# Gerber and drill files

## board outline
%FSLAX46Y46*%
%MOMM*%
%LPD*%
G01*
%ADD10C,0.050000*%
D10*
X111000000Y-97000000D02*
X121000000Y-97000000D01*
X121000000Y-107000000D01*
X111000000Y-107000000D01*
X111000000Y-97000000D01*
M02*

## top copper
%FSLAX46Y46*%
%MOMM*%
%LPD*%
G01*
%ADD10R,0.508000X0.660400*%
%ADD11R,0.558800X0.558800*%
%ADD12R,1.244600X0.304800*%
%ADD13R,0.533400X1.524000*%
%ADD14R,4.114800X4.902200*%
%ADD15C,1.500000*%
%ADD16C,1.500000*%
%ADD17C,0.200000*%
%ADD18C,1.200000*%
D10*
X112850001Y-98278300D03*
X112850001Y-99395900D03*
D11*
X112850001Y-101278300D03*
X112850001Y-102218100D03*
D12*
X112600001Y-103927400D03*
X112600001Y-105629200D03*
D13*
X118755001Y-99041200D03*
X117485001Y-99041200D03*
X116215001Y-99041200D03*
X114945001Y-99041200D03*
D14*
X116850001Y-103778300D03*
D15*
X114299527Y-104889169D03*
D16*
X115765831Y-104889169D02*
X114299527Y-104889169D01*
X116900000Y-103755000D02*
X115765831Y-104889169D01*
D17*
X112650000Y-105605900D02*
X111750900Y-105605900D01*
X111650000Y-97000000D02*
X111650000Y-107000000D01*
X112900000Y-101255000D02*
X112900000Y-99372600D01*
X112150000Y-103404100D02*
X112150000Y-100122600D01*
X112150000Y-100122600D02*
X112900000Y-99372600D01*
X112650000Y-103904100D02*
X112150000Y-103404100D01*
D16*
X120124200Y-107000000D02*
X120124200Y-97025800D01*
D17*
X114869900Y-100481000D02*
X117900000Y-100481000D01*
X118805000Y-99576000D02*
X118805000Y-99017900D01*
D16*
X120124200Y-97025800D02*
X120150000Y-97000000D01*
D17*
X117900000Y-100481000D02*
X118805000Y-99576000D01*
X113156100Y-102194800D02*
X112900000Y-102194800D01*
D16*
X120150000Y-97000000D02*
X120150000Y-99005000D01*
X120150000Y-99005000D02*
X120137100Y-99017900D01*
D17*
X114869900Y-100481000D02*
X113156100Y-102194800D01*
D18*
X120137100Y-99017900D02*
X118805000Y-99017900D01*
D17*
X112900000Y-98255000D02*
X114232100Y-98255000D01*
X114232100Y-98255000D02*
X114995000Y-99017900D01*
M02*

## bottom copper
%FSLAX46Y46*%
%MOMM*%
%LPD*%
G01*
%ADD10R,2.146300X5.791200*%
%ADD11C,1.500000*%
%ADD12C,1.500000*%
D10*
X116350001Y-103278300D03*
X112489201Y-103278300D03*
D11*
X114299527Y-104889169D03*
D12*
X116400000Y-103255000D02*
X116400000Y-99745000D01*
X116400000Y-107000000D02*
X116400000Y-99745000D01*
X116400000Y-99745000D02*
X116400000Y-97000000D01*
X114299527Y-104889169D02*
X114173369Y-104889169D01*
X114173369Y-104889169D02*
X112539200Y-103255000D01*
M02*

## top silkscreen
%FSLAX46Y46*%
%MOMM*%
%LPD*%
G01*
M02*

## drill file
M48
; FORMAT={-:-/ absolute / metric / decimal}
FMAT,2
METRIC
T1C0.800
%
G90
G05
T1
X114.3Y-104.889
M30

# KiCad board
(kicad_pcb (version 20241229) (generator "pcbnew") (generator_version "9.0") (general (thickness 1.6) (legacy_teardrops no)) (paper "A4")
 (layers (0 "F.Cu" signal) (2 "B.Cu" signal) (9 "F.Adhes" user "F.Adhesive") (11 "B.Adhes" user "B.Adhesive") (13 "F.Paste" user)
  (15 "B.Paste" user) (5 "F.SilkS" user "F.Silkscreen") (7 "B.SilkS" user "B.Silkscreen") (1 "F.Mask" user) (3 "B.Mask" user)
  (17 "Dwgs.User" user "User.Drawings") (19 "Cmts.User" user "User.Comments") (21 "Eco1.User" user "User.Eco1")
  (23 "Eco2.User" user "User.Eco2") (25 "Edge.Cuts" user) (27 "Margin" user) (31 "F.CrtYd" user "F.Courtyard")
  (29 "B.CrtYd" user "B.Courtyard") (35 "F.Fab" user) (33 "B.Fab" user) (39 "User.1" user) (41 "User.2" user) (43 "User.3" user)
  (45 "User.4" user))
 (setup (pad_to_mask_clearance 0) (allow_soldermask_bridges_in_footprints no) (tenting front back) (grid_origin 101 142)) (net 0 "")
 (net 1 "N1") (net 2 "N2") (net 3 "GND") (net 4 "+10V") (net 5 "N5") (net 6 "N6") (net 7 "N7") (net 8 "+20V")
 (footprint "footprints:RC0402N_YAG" (layer "F.Cu") (at 112.850001 98.8371 -90)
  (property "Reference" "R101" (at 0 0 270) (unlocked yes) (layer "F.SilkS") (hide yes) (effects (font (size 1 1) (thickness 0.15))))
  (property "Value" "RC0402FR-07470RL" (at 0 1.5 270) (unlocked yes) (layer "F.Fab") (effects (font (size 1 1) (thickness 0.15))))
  (pad "1" smd rect (at -0.5588 0 270) (size 0.6604 0.508) (layers "F.Cu" "F.Mask" "F.Paste") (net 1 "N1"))
  (pad "2" smd rect (at 0.5588 0 270) (size 0.6604 0.508) (layers "F.Cu" "F.Mask" "F.Paste") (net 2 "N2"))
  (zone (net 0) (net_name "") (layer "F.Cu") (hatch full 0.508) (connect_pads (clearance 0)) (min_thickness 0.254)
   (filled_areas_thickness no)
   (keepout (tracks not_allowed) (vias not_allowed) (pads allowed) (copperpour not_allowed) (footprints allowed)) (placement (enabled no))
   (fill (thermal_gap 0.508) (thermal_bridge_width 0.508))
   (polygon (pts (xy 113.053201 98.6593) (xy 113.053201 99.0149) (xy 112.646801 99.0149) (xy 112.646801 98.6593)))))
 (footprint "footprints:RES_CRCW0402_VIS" (layer "F.Cu") (at 112.850001 101.7482 -90)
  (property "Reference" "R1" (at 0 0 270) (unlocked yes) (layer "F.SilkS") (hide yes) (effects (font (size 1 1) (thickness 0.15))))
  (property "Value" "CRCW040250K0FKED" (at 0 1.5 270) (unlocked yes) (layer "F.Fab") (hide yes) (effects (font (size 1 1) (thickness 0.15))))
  (pad "1" smd rect (at -0.4699 0 270) (size 0.5588 0.5588) (layers "F.Cu" "F.Mask" "F.Paste") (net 2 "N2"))
  (pad "2" smd rect (at 0.4699 0 270) (size 0.5588 0.5588) (layers "F.Cu" "F.Mask" "F.Paste") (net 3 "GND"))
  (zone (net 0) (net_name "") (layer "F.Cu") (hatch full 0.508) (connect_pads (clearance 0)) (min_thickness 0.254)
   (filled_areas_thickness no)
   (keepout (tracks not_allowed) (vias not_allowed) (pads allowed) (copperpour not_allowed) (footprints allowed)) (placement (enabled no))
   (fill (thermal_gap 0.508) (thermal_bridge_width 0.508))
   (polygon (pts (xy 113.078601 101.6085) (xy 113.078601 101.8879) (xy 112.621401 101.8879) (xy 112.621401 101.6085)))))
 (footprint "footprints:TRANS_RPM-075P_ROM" (layer "F.Cu") (at 112.600001 104.7783 -90)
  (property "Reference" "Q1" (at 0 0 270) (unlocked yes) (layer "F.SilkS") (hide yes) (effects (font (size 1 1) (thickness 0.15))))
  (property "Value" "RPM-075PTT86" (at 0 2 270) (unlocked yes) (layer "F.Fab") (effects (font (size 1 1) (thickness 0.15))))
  (pad "1" smd rect (at -0.8509 0 270) (size 0.3048 1.2446) (layers "F.Cu" "F.Mask" "F.Paste") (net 2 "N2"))
  (pad "2" smd rect (at 0.8509 0 270) (size 0.3048 1.2446) (layers "F.Cu" "F.Mask" "F.Paste") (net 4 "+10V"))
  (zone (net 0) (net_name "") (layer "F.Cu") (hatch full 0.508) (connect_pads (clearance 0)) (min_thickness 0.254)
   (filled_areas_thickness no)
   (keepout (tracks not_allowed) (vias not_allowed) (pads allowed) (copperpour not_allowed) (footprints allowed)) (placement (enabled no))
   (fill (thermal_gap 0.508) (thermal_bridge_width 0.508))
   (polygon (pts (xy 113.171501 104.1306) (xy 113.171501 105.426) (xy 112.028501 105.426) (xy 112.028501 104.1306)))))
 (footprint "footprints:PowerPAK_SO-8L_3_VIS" (layer "F.Cu") (at 116.850001 102.648 180)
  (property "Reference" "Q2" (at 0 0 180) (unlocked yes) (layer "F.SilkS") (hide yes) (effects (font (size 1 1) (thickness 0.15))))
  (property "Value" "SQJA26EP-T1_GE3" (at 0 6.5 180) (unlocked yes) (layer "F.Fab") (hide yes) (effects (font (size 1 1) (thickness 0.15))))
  (pad "1" smd rect (at -1.905 3.6068 180) (size 0.5334 1.524) (layers "F.Cu" "F.Mask" "F.Paste") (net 3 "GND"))
  (pad "2" smd rect (at -0.635 3.6068 180) (size 0.5334 1.524) (layers "F.Cu" "F.Mask" "F.Paste") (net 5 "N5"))
  (pad "3" smd rect (at 0.635 3.6068 180) (size 0.5334 1.524) (layers "F.Cu" "F.Mask" "F.Paste") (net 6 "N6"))
  (pad "4" smd rect (at 1.905 3.6068 180) (size 0.5334 1.524) (layers "F.Cu" "F.Mask" "F.Paste") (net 1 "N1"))
  (pad "5" smd rect (at 0 -1.1303 180) (size 4.1148 4.9022) (layers "F.Cu" "F.Mask" "F.Paste") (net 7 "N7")))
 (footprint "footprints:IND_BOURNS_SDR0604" (layer "B.Cu") (at 114.419601 103.2783 180)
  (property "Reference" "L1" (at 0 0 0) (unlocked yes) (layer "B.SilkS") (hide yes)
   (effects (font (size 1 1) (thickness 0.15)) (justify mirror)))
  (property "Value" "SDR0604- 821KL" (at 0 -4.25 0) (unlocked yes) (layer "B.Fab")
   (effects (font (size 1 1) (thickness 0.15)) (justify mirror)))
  (pad "1" smd rect (at -1.9304 0 180) (size 2.1463 5.7912) (layers "B.Cu" "B.Mask" "B.Paste") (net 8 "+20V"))
  (pad "2" smd rect (at 1.9304 0 180) (size 2.1463 5.7912) (layers "B.Cu" "B.Mask" "B.Paste") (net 7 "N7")))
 (gr_rect (start 111 97) (end 121 107) (stroke (width 0.05) (type default)) (fill no) (layer "Edge.Cuts"))
 (segment (start 116.4 103.255) (end 116.4 99.745) (width 1.5) (layer "B.Cu") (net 8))
 (segment (start 116.4 107) (end 116.4 99.745) (width 1.5) (layer "B.Cu") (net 8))
 (segment (start 116.4 99.745) (end 116.4 97) (width 1.5) (layer "B.Cu") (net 8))
 (segment (start 115.765831 104.889169) (end 114.299527 104.889169) (width 1.5) (layer "F.Cu") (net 7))
 (segment (start 116.9 103.755) (end 115.765831 104.889169) (width 1.5) (layer "F.Cu") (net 7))
 (via (at 114.299527 104.889169) (size 1.5) (drill 0.8) (layers "F.Cu" "B.Cu") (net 7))
 (segment (start 114.299527 104.889169) (end 114.173369 104.889169) (width 1.5) (layer "B.Cu") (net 7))
 (segment (start 114.173369 104.889169) (end 112.5392 103.255) (width 1.5) (layer "B.Cu") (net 7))
 (segment (start 112.65 105.6059) (end 111.7509 105.6059) (width 0.2) (layer "F.Cu") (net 4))
 (segment (start 111.65 97) (end 111.65 107) (width 0.2) (layer "F.Cu") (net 4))
 (segment (start 112.9 101.255) (end 112.9 99.3726) (width 0.2) (layer "F.Cu") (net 2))
 (segment (start 112.15 103.4041) (end 112.15 100.1226) (width 0.2) (layer "F.Cu") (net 2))
 (segment (start 112.15 100.1226) (end 112.9 99.3726) (width 0.2) (layer "F.Cu") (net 2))
 (segment (start 112.65 103.9041) (end 112.15 103.4041) (width 0.2) (layer "F.Cu") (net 2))
 (segment (start 120.1242 107) (end 120.1242 97.0258) (width 1.5) (layer "F.Cu") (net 3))
 (segment (start 114.8699 100.481) (end 117.9 100.481) (width 0.2) (layer "F.Cu") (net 3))
 (segment (start 118.805 99.576) (end 118.805 99.0179) (width 0.2) (layer "F.Cu") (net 3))
 (segment (start 120.1242 97.0258) (end 120.15 97) (width 1.5) (layer "F.Cu") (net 3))
 (segment (start 117.9 100.481) (end 118.805 99.576) (width 0.2) (layer "F.Cu") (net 3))
 (segment (start 113.1561 102.1948) (end 112.9 102.1948) (width 0.2) (layer "F.Cu") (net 3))
 (segment (start 120.15 97) (end 120.15 99.005) (width 1.5) (layer "F.Cu") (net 3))
 (segment (start 120.15 99.005) (end 120.1371 99.0179) (width 1.5) (layer "F.Cu") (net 3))
 (segment (start 114.8699 100.481) (end 113.1561 102.1948) (width 0.2) (layer "F.Cu") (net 3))
 (segment (start 120.1371 99.0179) (end 118.805 99.0179) (width 1.2) (layer "F.Cu") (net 3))
 (segment (start 112.9 98.255) (end 114.2321 98.255) (width 0.2) (layer "F.Cu") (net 1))
 (segment (start 114.2321 98.255) (end 114.995 99.0179) (width 0.2) (layer "F.Cu") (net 1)))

